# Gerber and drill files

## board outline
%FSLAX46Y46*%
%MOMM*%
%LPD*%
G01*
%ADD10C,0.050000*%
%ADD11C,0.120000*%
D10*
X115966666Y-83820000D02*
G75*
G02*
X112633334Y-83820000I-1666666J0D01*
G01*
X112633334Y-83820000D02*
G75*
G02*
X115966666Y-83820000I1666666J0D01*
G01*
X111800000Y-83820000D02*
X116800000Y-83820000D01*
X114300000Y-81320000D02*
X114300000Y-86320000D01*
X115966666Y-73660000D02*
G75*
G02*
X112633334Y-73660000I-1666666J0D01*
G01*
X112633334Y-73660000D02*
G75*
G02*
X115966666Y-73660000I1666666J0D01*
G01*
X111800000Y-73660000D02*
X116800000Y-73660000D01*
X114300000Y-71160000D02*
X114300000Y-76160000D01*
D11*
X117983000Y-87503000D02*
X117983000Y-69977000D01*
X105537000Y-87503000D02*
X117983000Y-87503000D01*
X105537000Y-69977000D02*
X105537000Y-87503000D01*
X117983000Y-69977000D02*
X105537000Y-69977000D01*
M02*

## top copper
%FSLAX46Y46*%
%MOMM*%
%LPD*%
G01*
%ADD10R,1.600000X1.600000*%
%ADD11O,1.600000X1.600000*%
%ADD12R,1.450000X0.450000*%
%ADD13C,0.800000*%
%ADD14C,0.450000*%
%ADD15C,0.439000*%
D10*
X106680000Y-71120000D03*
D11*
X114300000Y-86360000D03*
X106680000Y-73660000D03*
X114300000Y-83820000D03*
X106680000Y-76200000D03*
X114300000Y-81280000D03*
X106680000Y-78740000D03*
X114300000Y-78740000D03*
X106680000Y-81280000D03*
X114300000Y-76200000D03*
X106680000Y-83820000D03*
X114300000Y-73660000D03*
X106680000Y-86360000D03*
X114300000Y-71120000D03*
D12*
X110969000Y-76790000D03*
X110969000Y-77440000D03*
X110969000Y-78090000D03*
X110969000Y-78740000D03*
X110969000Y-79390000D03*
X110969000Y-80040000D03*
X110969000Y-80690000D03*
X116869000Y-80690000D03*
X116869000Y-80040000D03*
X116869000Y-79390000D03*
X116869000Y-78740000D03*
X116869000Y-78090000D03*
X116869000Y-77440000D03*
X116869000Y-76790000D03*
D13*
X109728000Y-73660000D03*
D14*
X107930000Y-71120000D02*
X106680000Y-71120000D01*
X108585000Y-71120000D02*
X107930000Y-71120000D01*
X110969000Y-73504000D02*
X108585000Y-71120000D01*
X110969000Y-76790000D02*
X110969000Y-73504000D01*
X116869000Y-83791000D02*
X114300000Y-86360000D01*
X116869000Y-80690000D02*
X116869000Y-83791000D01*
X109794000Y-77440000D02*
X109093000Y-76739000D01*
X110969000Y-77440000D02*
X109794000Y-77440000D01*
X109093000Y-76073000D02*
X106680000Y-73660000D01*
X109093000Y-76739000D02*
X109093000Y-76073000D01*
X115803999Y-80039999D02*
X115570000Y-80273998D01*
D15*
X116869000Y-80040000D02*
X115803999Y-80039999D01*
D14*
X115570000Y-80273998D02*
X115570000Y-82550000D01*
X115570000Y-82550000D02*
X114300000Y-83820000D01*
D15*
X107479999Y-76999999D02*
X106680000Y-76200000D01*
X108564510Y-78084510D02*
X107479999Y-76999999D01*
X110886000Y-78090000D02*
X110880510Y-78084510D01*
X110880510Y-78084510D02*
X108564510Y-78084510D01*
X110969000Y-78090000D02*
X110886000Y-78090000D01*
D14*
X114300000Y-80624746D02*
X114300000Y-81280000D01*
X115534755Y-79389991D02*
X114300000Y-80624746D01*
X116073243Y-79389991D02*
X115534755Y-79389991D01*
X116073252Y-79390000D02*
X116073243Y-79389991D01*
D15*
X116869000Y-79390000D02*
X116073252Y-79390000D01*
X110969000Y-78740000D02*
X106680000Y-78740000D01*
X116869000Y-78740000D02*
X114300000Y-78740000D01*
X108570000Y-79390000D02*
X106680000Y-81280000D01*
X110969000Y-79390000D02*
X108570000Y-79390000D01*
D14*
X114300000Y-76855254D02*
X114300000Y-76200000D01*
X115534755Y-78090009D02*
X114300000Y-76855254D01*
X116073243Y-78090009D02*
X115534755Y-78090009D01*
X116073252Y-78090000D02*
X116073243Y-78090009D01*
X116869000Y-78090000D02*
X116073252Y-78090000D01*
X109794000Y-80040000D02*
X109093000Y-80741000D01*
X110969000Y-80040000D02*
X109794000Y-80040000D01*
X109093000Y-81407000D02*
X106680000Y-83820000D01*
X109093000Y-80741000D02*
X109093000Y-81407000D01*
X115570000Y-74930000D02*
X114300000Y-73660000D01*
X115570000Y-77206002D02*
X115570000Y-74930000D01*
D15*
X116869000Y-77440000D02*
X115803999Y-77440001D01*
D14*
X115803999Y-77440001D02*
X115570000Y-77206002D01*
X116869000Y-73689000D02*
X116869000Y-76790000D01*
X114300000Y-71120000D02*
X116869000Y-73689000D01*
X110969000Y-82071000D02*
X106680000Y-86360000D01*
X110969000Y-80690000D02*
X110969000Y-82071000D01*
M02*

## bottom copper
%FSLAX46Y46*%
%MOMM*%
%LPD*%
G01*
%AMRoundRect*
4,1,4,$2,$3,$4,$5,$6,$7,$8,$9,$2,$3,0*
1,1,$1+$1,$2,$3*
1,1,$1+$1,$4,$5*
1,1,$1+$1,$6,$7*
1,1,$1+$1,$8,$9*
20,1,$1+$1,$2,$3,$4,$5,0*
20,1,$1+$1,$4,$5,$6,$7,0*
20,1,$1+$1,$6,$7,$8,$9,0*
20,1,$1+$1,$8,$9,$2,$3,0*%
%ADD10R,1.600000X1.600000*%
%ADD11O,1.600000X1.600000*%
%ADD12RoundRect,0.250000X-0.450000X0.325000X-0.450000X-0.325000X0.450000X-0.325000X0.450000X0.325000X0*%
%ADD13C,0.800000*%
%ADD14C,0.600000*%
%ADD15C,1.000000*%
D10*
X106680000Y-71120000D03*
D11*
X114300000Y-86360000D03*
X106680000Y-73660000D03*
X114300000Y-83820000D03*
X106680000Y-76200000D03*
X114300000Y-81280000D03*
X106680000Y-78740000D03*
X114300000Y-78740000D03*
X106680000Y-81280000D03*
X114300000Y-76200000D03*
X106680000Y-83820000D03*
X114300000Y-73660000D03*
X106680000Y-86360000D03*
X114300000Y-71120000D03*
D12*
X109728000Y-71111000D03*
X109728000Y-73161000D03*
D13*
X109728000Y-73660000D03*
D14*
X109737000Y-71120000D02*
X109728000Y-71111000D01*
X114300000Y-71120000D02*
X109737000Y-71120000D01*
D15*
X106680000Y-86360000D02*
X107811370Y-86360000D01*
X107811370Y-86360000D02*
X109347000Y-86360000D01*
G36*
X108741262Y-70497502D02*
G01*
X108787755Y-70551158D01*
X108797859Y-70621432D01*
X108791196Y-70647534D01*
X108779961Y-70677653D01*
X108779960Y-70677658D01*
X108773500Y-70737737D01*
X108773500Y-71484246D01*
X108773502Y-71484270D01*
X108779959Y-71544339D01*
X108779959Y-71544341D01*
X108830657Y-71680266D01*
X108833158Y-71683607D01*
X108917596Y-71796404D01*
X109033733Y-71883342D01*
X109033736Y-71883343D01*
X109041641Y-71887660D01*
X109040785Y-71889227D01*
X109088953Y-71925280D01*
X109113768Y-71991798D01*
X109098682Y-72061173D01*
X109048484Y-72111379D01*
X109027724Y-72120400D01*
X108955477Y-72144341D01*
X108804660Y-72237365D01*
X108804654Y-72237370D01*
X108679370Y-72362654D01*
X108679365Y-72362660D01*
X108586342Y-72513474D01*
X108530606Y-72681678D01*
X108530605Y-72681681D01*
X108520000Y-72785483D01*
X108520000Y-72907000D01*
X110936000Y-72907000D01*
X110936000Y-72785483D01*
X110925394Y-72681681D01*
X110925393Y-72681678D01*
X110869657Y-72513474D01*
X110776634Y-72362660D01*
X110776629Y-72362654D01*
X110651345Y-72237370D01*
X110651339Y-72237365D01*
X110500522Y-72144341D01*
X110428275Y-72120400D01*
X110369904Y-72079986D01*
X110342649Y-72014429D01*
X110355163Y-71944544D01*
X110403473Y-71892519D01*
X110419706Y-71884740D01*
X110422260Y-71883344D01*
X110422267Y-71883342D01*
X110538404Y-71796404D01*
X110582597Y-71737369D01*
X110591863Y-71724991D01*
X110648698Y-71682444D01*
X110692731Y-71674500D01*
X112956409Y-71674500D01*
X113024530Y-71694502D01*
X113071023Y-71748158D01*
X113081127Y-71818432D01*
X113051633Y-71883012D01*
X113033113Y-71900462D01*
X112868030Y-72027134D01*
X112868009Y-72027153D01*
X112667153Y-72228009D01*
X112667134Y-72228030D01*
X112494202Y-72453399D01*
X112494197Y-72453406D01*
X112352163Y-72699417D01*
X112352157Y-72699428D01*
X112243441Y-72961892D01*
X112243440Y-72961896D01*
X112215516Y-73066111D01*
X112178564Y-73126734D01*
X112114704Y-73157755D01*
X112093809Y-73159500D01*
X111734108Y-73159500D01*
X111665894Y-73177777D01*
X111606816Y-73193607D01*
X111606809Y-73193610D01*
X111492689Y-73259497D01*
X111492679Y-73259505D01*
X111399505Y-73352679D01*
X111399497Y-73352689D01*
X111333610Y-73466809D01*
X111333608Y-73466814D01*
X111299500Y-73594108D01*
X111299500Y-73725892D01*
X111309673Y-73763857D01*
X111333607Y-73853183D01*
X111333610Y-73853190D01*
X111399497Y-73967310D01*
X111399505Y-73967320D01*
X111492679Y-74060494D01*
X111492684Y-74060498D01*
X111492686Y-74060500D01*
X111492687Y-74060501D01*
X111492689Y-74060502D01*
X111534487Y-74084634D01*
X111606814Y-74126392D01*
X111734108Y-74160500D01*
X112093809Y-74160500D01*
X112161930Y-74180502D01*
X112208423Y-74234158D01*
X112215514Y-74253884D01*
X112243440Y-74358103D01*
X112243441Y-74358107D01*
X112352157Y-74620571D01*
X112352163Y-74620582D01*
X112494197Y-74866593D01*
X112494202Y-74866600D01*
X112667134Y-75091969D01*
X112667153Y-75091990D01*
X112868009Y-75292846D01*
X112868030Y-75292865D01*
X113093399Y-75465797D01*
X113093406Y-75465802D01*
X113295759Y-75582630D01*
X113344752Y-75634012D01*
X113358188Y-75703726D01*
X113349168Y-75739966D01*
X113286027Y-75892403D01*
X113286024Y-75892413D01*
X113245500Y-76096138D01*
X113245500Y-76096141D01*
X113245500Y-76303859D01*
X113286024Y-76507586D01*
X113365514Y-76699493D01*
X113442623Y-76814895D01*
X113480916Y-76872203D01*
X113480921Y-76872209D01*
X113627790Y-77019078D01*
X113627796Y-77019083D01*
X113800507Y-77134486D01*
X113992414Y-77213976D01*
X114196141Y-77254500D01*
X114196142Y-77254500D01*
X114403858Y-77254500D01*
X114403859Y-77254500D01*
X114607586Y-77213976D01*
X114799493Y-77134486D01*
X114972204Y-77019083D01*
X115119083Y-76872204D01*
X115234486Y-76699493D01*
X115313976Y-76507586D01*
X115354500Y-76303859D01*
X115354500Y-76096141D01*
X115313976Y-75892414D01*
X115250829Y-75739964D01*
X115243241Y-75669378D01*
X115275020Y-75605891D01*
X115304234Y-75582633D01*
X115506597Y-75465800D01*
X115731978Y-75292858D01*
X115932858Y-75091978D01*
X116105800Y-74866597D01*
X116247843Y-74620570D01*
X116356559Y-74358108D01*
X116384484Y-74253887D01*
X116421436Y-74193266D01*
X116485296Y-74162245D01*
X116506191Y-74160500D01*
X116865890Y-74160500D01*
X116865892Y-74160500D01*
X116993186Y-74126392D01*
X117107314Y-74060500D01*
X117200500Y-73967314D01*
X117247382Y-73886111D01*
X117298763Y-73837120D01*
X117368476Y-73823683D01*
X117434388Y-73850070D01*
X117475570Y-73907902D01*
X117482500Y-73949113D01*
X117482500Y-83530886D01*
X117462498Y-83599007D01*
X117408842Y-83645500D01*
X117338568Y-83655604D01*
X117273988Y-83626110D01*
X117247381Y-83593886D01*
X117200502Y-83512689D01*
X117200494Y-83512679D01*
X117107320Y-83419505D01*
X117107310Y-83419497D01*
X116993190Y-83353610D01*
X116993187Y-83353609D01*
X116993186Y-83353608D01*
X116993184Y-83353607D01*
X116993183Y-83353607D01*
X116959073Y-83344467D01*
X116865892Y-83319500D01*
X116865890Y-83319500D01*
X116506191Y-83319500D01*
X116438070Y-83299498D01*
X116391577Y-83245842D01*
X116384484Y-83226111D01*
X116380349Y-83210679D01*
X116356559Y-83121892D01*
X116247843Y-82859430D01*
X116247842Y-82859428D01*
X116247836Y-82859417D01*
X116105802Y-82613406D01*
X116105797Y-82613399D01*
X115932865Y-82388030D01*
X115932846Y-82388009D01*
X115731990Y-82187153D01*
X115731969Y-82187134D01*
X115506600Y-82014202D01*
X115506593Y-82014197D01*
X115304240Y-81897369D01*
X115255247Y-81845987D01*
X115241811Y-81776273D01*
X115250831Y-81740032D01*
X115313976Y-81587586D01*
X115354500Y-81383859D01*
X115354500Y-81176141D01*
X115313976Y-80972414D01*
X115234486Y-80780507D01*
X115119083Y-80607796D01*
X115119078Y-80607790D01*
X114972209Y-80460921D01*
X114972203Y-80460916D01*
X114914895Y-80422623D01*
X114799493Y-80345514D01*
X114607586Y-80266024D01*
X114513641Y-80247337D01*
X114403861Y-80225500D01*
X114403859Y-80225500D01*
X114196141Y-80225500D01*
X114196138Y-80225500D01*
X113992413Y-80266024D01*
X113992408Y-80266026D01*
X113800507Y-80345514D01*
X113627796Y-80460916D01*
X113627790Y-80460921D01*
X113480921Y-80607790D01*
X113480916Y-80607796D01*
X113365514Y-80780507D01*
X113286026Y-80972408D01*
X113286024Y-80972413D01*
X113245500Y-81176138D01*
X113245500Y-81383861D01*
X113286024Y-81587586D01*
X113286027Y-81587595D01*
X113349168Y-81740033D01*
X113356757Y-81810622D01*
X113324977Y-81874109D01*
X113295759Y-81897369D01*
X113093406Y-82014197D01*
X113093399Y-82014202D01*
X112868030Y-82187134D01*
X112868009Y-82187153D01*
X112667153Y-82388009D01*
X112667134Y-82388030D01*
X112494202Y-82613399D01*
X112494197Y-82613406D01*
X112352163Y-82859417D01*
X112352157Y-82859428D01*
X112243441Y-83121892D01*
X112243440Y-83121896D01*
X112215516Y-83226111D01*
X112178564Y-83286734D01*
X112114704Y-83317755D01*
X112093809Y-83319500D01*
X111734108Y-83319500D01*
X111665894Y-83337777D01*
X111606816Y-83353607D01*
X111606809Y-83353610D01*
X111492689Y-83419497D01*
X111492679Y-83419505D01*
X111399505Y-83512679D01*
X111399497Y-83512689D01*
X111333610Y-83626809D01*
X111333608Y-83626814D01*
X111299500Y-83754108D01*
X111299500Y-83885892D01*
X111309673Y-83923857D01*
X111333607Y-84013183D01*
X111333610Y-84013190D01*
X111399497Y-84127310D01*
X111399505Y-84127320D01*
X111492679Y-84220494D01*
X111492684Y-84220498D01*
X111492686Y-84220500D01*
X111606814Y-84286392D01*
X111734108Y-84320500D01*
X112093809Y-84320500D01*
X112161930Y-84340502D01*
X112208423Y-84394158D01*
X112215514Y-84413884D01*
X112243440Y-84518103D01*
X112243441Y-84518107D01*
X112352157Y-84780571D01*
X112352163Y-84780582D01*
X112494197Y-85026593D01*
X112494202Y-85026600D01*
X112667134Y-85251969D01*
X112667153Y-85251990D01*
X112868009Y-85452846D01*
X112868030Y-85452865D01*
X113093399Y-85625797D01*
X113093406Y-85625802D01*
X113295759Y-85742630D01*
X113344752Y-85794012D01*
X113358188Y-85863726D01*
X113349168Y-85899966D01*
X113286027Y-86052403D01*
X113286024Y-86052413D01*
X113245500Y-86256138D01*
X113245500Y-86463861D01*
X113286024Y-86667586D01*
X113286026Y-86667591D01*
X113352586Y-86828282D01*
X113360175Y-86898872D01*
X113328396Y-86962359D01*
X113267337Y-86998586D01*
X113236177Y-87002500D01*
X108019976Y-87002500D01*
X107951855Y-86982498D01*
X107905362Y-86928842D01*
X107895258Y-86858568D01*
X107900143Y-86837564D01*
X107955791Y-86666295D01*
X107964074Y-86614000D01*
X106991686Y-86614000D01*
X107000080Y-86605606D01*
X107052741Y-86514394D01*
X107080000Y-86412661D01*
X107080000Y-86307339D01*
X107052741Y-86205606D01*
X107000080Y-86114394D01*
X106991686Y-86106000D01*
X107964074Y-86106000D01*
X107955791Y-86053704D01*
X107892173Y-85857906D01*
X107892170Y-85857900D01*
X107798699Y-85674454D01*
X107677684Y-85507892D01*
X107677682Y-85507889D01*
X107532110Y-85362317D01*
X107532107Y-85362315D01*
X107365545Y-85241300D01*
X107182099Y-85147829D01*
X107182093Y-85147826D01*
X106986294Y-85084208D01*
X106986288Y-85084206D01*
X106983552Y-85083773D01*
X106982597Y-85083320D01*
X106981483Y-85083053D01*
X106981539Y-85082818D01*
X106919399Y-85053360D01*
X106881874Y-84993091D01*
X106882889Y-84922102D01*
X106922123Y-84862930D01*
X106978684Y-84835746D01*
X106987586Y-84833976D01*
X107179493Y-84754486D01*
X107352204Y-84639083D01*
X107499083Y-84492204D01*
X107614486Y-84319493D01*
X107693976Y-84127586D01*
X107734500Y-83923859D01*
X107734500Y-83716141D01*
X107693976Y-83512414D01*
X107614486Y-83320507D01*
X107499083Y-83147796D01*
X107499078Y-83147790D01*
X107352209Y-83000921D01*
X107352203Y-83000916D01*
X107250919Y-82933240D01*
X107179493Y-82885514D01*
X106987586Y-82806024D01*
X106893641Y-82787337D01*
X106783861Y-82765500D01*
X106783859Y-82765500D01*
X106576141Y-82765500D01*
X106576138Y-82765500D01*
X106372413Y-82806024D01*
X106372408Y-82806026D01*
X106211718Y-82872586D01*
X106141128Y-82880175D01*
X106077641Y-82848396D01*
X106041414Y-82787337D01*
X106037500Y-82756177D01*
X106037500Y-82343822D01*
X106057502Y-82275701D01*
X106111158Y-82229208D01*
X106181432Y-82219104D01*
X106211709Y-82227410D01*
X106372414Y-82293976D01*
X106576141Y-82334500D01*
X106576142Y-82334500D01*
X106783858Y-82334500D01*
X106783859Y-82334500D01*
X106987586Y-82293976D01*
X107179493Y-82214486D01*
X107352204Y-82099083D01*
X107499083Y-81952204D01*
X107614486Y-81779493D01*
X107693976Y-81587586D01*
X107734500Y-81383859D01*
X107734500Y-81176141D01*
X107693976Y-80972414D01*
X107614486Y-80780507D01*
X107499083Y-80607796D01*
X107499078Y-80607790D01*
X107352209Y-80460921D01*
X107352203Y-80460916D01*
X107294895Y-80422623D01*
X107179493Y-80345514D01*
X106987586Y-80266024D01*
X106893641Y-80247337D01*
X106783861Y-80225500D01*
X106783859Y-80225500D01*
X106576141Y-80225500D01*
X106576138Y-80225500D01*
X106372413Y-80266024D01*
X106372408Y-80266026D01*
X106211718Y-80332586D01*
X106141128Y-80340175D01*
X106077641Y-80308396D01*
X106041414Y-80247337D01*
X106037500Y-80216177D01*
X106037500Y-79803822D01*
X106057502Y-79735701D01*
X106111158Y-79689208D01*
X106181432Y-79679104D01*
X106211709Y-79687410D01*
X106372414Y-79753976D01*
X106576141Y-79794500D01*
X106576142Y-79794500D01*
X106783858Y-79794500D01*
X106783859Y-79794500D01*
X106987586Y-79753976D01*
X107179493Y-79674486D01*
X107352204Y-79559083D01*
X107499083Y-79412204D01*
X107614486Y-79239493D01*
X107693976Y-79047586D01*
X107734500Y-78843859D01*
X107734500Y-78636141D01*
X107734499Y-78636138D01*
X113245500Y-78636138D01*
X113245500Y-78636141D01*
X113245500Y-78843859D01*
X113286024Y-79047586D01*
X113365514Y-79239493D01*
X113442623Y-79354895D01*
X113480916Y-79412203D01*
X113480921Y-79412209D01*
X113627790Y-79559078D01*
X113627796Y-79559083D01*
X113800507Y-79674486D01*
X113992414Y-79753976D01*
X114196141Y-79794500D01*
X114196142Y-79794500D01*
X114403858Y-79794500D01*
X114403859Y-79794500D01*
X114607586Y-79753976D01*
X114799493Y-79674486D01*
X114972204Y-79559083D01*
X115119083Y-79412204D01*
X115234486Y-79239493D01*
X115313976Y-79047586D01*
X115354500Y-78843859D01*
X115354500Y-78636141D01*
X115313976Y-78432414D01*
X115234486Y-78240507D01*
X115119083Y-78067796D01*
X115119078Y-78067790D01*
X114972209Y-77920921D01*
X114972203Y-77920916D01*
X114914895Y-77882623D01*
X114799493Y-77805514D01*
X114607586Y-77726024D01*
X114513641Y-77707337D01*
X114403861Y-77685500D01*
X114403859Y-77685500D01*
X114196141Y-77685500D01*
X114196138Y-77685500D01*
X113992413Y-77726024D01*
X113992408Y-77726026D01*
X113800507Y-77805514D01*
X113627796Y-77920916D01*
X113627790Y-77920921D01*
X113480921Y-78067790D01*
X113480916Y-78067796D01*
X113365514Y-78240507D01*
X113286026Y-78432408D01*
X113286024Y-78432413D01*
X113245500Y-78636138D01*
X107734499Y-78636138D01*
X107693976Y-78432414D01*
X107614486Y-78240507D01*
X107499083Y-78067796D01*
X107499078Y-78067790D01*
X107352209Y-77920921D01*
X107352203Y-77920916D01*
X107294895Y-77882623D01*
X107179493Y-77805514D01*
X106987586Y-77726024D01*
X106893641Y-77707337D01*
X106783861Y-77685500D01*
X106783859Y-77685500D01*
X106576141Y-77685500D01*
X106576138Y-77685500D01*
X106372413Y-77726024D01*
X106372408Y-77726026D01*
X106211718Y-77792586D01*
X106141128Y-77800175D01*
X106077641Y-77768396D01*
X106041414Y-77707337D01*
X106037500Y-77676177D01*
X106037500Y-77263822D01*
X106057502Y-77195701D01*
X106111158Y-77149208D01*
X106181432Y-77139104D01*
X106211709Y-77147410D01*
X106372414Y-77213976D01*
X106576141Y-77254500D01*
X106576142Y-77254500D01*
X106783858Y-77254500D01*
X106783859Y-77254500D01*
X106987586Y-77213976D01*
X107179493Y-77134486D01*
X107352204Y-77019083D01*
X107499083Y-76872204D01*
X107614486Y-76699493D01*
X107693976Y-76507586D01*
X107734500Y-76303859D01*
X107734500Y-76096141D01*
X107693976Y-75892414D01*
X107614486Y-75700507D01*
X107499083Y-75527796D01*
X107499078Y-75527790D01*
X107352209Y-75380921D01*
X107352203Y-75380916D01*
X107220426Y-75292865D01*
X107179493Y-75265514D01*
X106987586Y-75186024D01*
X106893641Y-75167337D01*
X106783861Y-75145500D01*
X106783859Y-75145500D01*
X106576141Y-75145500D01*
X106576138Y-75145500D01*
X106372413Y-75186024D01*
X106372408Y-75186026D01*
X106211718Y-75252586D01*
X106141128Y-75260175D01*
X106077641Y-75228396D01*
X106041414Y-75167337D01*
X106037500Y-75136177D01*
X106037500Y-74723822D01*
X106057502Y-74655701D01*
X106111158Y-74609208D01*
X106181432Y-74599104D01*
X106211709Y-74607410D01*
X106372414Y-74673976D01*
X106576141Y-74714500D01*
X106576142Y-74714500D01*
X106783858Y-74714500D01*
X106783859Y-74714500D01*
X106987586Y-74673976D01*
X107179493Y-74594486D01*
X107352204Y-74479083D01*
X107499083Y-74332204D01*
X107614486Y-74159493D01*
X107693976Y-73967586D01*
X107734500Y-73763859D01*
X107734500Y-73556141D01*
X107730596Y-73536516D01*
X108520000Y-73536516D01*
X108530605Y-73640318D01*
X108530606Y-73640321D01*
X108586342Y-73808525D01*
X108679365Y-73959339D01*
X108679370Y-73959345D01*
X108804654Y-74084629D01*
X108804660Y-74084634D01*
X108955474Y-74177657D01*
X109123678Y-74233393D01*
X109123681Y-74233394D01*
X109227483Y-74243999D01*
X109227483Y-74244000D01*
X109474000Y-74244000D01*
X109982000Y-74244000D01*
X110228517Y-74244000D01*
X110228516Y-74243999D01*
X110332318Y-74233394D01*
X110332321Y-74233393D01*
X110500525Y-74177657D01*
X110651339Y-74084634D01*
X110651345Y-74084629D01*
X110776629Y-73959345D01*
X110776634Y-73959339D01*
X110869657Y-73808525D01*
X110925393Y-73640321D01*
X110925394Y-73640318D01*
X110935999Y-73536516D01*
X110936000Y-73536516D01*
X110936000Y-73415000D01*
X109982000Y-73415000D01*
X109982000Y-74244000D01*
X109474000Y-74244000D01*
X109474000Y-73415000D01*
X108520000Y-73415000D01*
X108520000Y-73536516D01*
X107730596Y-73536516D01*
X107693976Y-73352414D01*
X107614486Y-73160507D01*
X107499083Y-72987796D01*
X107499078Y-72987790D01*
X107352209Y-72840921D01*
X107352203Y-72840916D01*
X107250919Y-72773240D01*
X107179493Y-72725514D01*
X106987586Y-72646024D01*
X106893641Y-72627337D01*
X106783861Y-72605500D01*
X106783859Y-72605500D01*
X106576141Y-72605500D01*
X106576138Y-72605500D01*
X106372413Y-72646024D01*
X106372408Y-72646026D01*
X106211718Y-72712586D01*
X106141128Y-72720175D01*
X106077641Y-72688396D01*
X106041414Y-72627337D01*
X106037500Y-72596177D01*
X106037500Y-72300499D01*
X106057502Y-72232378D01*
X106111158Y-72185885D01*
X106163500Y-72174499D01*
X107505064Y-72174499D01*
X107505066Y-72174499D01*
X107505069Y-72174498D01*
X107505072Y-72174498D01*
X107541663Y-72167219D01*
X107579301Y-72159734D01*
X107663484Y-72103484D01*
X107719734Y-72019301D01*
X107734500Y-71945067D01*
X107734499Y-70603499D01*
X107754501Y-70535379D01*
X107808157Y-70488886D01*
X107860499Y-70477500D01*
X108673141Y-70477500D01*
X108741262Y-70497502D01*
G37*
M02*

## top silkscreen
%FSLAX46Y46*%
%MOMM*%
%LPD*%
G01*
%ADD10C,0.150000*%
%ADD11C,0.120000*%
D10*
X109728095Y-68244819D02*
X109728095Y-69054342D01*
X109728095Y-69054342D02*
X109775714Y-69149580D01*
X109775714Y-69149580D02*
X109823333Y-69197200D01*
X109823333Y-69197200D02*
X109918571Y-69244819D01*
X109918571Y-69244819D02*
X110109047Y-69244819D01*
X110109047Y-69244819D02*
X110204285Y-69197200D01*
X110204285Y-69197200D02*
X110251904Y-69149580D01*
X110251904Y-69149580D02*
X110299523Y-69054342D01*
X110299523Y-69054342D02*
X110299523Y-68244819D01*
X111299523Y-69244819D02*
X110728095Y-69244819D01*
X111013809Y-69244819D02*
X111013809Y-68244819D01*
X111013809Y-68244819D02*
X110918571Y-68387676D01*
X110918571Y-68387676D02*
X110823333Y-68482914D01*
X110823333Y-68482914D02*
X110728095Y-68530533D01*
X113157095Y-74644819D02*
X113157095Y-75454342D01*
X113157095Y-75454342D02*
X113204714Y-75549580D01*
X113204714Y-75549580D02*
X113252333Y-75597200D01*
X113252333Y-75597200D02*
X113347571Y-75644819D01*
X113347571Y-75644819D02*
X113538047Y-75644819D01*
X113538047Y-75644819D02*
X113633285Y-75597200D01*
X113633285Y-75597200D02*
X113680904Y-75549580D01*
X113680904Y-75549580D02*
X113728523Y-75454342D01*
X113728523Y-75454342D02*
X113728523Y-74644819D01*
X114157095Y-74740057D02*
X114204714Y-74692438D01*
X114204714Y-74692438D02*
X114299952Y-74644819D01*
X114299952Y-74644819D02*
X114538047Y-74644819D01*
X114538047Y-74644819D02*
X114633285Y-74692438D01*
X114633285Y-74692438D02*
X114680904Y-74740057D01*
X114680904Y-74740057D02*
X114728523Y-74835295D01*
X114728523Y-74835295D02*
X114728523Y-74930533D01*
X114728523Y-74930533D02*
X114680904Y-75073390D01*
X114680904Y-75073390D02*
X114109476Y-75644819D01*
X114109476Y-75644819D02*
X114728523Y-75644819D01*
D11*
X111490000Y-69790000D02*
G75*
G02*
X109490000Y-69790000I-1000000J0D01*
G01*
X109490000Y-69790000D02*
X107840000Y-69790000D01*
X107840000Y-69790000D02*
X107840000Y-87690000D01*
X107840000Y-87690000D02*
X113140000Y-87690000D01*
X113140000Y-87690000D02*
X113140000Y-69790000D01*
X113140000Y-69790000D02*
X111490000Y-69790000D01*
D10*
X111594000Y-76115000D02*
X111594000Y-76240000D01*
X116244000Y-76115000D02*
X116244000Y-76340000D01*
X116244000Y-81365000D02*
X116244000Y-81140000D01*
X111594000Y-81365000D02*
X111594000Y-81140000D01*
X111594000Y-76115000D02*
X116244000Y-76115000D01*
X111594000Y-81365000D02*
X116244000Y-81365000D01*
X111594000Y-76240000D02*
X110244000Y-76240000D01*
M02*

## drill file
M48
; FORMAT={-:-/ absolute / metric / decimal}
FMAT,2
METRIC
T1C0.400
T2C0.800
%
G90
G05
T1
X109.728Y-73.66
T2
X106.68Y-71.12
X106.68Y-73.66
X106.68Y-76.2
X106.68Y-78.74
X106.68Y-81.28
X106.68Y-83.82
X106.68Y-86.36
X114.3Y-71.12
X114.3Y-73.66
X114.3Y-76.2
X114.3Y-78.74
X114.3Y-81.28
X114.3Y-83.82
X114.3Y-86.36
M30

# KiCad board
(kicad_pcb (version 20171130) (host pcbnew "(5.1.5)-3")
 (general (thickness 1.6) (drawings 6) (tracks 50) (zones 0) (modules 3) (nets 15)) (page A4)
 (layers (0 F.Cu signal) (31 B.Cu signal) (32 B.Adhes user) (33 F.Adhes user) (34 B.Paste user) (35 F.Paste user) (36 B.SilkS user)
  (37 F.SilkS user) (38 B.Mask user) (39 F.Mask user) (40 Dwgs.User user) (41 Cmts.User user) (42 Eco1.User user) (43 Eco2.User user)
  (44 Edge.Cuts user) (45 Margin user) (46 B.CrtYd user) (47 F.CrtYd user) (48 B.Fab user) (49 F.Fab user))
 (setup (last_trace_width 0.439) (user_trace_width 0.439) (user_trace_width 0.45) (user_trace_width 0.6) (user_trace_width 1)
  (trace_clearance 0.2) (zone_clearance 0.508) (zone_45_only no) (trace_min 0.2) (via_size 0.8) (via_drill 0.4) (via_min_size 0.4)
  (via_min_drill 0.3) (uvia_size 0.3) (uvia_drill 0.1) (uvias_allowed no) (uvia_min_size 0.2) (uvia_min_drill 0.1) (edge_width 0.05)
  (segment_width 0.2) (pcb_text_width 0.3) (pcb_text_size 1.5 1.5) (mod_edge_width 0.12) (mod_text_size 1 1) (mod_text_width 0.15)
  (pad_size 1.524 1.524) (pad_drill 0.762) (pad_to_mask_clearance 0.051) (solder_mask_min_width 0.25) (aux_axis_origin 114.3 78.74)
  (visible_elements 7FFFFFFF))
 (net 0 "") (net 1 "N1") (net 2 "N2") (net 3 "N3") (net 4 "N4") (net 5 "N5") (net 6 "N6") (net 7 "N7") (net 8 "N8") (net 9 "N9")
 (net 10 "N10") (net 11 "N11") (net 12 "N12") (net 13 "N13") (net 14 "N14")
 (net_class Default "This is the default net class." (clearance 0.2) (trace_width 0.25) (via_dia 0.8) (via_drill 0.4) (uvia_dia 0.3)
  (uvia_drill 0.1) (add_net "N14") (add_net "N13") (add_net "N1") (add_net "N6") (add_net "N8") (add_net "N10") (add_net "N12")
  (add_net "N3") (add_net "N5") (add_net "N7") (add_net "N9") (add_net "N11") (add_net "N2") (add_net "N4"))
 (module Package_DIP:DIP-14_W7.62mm (layer F.Cu) (at 106.68 71.12)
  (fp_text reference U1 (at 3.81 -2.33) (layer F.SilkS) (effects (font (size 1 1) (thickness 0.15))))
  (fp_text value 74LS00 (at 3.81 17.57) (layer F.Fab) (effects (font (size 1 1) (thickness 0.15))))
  (fp_arc (start 3.81 -1.33) (end 2.81 -1.33) (angle -180) (layer F.SilkS) (width 0.12))
  (fp_line (start 2.81 -1.33) (end 1.16 -1.33) (layer F.SilkS) (width 0.12))
  (fp_line (start 1.16 -1.33) (end 1.16 16.57) (layer F.SilkS) (width 0.12))
  (fp_line (start 1.16 16.57) (end 6.46 16.57) (layer F.SilkS) (width 0.12))
  (fp_line (start 6.46 16.57) (end 6.46 -1.33) (layer F.SilkS) (width 0.12))
  (fp_line (start 6.46 -1.33) (end 4.81 -1.33) (layer F.SilkS) (width 0.12))
  (pad 1 thru_hole rect (at 0 0) (size 1.6 1.6) (drill 0.8) (layers *.Cu *.Mask) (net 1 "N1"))
  (pad 8 thru_hole oval (at 7.62 15.24) (size 1.6 1.6) (drill 0.8) (layers *.Cu *.Mask) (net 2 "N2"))
  (pad 2 thru_hole oval (at 0 2.54) (size 1.6 1.6) (drill 0.8) (layers *.Cu *.Mask) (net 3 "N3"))
  (pad 9 thru_hole oval (at 7.62 12.7) (size 1.6 1.6) (drill 0.8) (layers *.Cu *.Mask) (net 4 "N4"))
  (pad 3 thru_hole oval (at 0 5.08) (size 1.6 1.6) (drill 0.8) (layers *.Cu *.Mask) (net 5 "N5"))
  (pad 10 thru_hole oval (at 7.62 10.16) (size 1.6 1.6) (drill 0.8) (layers *.Cu *.Mask) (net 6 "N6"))
  (pad 4 thru_hole oval (at 0 7.62) (size 1.6 1.6) (drill 0.8) (layers *.Cu *.Mask) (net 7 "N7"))
  (pad 11 thru_hole oval (at 7.62 7.62) (size 1.6 1.6) (drill 0.8) (layers *.Cu *.Mask) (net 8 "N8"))
  (pad 5 thru_hole oval (at 0 10.16) (size 1.6 1.6) (drill 0.8) (layers *.Cu *.Mask) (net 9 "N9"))
  (pad 12 thru_hole oval (at 7.62 5.08) (size 1.6 1.6) (drill 0.8) (layers *.Cu *.Mask) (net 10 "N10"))
  (pad 6 thru_hole oval (at 0 12.7) (size 1.6 1.6) (drill 0.8) (layers *.Cu *.Mask) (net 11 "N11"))
  (pad 13 thru_hole oval (at 7.62 2.54) (size 1.6 1.6) (drill 0.8) (layers *.Cu *.Mask) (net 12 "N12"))
  (pad 7 thru_hole oval (at 0 15.24) (size 1.6 1.6) (drill 0.8) (layers *.Cu *.Mask) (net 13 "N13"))
  (pad 14 thru_hole oval (at 7.62 0) (size 1.6 1.6) (drill 0.8) (layers *.Cu *.Mask) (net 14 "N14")))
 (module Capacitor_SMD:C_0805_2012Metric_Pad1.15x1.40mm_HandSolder (layer B.Cu) (at 109.728 72.136 270)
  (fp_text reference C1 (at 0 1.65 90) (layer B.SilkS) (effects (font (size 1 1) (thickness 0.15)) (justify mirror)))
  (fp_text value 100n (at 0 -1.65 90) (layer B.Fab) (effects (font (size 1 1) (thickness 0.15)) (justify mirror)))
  (pad 1 smd roundrect (at -1.025 0 270) (size 1.15 1.4) (layers B.Cu B.Paste B.Mask) (roundrect_rratio 0.217391) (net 14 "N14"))
  (pad 2 smd roundrect (at 1.025 0 270) (size 1.15 1.4) (layers B.Cu B.Paste B.Mask) (roundrect_rratio 0.217391) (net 13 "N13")))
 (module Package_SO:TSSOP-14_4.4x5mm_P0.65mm (layer F.Cu) (at 113.919 78.74)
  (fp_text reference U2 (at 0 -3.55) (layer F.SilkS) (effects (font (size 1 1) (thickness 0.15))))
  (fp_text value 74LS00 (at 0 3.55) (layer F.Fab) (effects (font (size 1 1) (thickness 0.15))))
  (fp_line (start -2.325 -2.625) (end -2.325 -2.5) (layer F.SilkS) (width 0.15))
  (fp_line (start 2.325 -2.625) (end 2.325 -2.4) (layer F.SilkS) (width 0.15))
  (fp_line (start 2.325 2.625) (end 2.325 2.4) (layer F.SilkS) (width 0.15))
  (fp_line (start -2.325 2.625) (end -2.325 2.4) (layer F.SilkS) (width 0.15))
  (fp_line (start -2.325 -2.625) (end 2.325 -2.625) (layer F.SilkS) (width 0.15))
  (fp_line (start -2.325 2.625) (end 2.325 2.625) (layer F.SilkS) (width 0.15))
  (fp_line (start -2.325 -2.5) (end -3.675 -2.5) (layer F.SilkS) (width 0.15))
  (pad 1 smd rect (at -2.95 -1.95) (size 1.45 0.45) (layers F.Cu F.Paste F.Mask) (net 1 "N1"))
  (pad 2 smd rect (at -2.95 -1.3) (size 1.45 0.45) (layers F.Cu F.Paste F.Mask) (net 3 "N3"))
  (pad 3 smd rect (at -2.95 -0.65) (size 1.45 0.45) (layers F.Cu F.Paste F.Mask) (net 5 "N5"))
  (pad 4 smd rect (at -2.95 0) (size 1.45 0.45) (layers F.Cu F.Paste F.Mask) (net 7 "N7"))
  (pad 5 smd rect (at -2.95 0.65) (size 1.45 0.45) (layers F.Cu F.Paste F.Mask) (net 9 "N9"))
  (pad 6 smd rect (at -2.95 1.3) (size 1.45 0.45) (layers F.Cu F.Paste F.Mask) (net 11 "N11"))
  (pad 7 smd rect (at -2.95 1.95) (size 1.45 0.45) (layers F.Cu F.Paste F.Mask) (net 13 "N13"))
  (pad 8 smd rect (at 2.95 1.95) (size 1.45 0.45) (layers F.Cu F.Paste F.Mask) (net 2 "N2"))
  (pad 9 smd rect (at 2.95 1.3) (size 1.45 0.45) (layers F.Cu F.Paste F.Mask) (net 4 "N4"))
  (pad 10 smd rect (at 2.95 0.65) (size 1.45 0.45) (layers F.Cu F.Paste F.Mask) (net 6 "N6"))
  (pad 11 smd rect (at 2.95 0) (size 1.45 0.45) (layers F.Cu F.Paste F.Mask) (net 8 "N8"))
  (pad 12 smd rect (at 2.95 -0.65) (size 1.45 0.45) (layers F.Cu F.Paste F.Mask) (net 10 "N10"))
  (pad 13 smd rect (at 2.95 -1.3) (size 1.45 0.45) (layers F.Cu F.Paste F.Mask) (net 12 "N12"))
  (pad 14 smd rect (at 2.95 -1.95) (size 1.45 0.45) (layers F.Cu F.Paste F.Mask) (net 14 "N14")))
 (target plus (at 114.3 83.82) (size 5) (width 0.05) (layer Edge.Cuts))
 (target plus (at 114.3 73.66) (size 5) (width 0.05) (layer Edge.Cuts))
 (gr_line (start 117.983 87.503) (end 117.983 69.977) (layer Edge.Cuts) (width 0.12))
 (gr_line (start 105.537 87.503) (end 117.983 87.503) (layer Edge.Cuts) (width 0.12))
 (gr_line (start 105.537 69.977) (end 105.537 87.503) (layer Edge.Cuts) (width 0.12))
 (gr_line (start 117.983 69.977) (end 105.537 69.977) (layer Edge.Cuts) (width 0.12))
 (segment (start 107.93 71.12) (end 106.68 71.12) (width 0.45) (layer F.Cu) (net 1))
 (segment (start 108.585 71.12) (end 107.93 71.12) (width 0.45) (layer F.Cu) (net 1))
 (segment (start 110.969 73.504) (end 108.585 71.12) (width 0.45) (layer F.Cu) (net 1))
 (segment (start 110.969 76.79) (end 110.969 73.504) (width 0.45) (layer F.Cu) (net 1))
 (segment (start 116.869 83.791) (end 114.3 86.36) (width 0.45) (layer F.Cu) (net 2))
 (segment (start 116.869 80.69) (end 116.869 83.791) (width 0.45) (layer F.Cu) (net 2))
 (segment (start 109.794 77.44) (end 109.093 76.739) (width 0.45) (layer F.Cu) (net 3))
 (segment (start 110.969 77.44) (end 109.794 77.44) (width 0.45) (layer F.Cu) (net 3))
 (segment (start 109.093 76.073) (end 106.68 73.66) (width 0.45) (layer F.Cu) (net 3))
 (segment (start 109.093 76.739) (end 109.093 76.073) (width 0.45) (layer F.Cu) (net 3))
 (segment (start 115.803999 80.039999) (end 115.57 80.273998) (width 0.45) (layer F.Cu) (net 4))
 (segment (start 116.869 80.04) (end 115.803999 80.039999) (width 0.439) (layer F.Cu) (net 4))
 (segment (start 115.57 80.273998) (end 115.57 82.55) (width 0.45) (layer F.Cu) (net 4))
 (segment (start 115.57 82.55) (end 114.3 83.82) (width 0.45) (layer F.Cu) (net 4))
 (segment (start 107.479999 76.999999) (end 106.68 76.2) (width 0.439) (layer F.Cu) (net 5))
 (segment (start 108.56451 78.08451) (end 107.479999 76.999999) (width 0.439) (layer F.Cu) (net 5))
 (segment (start 110.886 78.09) (end 110.88051 78.08451) (width 0.439) (layer F.Cu) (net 5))
 (segment (start 110.88051 78.08451) (end 108.56451 78.08451) (width 0.439) (layer F.Cu) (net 5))
 (segment (start 110.969 78.09) (end 110.886 78.09) (width 0.439) (layer F.Cu) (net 5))
 (segment (start 114.3 80.624746) (end 114.3 81.28) (width 0.45) (layer F.Cu) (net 6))
 (segment (start 115.534755 79.389991) (end 114.3 80.624746) (width 0.45) (layer F.Cu) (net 6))
 (segment (start 116.073243 79.389991) (end 115.534755 79.389991) (width 0.45) (layer F.Cu) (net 6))
 (segment (start 116.073252 79.39) (end 116.073243 79.389991) (width 0.45) (layer F.Cu) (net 6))
 (segment (start 116.869 79.39) (end 116.073252 79.39) (width 0.439) (layer F.Cu) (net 6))
 (segment (start 110.969 78.74) (end 106.68 78.74) (width 0.439) (layer F.Cu) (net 7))
 (segment (start 116.869 78.74) (end 114.3 78.74) (width 0.439) (layer F.Cu) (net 8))
 (segment (start 108.57 79.39) (end 106.68 81.28) (width 0.439) (layer F.Cu) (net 9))
 (segment (start 110.969 79.39) (end 108.57 79.39) (width 0.439) (layer F.Cu) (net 9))
 (segment (start 114.3 76.855254) (end 114.3 76.2) (width 0.45) (layer F.Cu) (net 10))
 (segment (start 115.534755 78.090009) (end 114.3 76.855254) (width 0.45) (layer F.Cu) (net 10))
 (segment (start 116.073243 78.090009) (end 115.534755 78.090009) (width 0.45) (layer F.Cu) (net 10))
 (segment (start 116.073252 78.09) (end 116.073243 78.090009) (width 0.45) (layer F.Cu) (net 10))
 (segment (start 116.869 78.09) (end 116.073252 78.09) (width 0.45) (layer F.Cu) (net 10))
 (segment (start 109.794 80.04) (end 109.093 80.741) (width 0.45) (layer F.Cu) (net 11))
 (segment (start 110.969 80.04) (end 109.794 80.04) (width 0.45) (layer F.Cu) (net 11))
 (segment (start 109.093 81.407) (end 106.68 83.82) (width 0.45) (layer F.Cu) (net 11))
 (segment (start 109.093 80.741) (end 109.093 81.407) (width 0.45) (layer F.Cu) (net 11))
 (segment (start 115.57 74.93) (end 114.3 73.66) (width 0.45) (layer F.Cu) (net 12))
 (segment (start 115.57 77.206002) (end 115.57 74.93) (width 0.45) (layer F.Cu) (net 12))
 (segment (start 116.869 77.44) (end 115.803999 77.440001) (width 0.439) (layer F.Cu) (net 12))
 (segment (start 115.803999 77.440001) (end 115.57 77.206002) (width 0.45) (layer F.Cu) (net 12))
 (segment (start 109.737 71.12) (end 109.728 71.111) (width 0.6) (layer B.Cu) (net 14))
 (segment (start 114.3 71.12) (end 109.737 71.12) (width 0.6) (layer B.Cu) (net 14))
 (segment (start 116.869 73.689) (end 116.869 76.79) (width 0.45) (layer F.Cu) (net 14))
 (segment (start 114.3 71.12) (end 116.869 73.689) (width 0.45) (layer F.Cu) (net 14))
 (via (at 109.728 73.66) (size 0.8) (drill 0.4) (layers F.Cu B.Cu) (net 13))
 (segment (start 110.969 82.071) (end 106.68 86.36) (width 0.45) (layer F.Cu) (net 13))
 (segment (start 110.969 80.69) (end 110.969 82.071) (width 0.45) (layer F.Cu) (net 13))
 (segment (start 106.68 86.36) (end 107.81137 86.36) (width 1) (layer B.Cu) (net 13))
 (segment (start 107.81137 86.36) (end 109.347 86.36) (width 1) (layer B.Cu) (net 13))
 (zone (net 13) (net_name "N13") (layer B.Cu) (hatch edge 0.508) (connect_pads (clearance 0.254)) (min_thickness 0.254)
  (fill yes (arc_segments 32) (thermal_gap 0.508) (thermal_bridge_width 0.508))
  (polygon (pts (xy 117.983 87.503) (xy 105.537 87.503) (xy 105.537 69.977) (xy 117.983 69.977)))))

